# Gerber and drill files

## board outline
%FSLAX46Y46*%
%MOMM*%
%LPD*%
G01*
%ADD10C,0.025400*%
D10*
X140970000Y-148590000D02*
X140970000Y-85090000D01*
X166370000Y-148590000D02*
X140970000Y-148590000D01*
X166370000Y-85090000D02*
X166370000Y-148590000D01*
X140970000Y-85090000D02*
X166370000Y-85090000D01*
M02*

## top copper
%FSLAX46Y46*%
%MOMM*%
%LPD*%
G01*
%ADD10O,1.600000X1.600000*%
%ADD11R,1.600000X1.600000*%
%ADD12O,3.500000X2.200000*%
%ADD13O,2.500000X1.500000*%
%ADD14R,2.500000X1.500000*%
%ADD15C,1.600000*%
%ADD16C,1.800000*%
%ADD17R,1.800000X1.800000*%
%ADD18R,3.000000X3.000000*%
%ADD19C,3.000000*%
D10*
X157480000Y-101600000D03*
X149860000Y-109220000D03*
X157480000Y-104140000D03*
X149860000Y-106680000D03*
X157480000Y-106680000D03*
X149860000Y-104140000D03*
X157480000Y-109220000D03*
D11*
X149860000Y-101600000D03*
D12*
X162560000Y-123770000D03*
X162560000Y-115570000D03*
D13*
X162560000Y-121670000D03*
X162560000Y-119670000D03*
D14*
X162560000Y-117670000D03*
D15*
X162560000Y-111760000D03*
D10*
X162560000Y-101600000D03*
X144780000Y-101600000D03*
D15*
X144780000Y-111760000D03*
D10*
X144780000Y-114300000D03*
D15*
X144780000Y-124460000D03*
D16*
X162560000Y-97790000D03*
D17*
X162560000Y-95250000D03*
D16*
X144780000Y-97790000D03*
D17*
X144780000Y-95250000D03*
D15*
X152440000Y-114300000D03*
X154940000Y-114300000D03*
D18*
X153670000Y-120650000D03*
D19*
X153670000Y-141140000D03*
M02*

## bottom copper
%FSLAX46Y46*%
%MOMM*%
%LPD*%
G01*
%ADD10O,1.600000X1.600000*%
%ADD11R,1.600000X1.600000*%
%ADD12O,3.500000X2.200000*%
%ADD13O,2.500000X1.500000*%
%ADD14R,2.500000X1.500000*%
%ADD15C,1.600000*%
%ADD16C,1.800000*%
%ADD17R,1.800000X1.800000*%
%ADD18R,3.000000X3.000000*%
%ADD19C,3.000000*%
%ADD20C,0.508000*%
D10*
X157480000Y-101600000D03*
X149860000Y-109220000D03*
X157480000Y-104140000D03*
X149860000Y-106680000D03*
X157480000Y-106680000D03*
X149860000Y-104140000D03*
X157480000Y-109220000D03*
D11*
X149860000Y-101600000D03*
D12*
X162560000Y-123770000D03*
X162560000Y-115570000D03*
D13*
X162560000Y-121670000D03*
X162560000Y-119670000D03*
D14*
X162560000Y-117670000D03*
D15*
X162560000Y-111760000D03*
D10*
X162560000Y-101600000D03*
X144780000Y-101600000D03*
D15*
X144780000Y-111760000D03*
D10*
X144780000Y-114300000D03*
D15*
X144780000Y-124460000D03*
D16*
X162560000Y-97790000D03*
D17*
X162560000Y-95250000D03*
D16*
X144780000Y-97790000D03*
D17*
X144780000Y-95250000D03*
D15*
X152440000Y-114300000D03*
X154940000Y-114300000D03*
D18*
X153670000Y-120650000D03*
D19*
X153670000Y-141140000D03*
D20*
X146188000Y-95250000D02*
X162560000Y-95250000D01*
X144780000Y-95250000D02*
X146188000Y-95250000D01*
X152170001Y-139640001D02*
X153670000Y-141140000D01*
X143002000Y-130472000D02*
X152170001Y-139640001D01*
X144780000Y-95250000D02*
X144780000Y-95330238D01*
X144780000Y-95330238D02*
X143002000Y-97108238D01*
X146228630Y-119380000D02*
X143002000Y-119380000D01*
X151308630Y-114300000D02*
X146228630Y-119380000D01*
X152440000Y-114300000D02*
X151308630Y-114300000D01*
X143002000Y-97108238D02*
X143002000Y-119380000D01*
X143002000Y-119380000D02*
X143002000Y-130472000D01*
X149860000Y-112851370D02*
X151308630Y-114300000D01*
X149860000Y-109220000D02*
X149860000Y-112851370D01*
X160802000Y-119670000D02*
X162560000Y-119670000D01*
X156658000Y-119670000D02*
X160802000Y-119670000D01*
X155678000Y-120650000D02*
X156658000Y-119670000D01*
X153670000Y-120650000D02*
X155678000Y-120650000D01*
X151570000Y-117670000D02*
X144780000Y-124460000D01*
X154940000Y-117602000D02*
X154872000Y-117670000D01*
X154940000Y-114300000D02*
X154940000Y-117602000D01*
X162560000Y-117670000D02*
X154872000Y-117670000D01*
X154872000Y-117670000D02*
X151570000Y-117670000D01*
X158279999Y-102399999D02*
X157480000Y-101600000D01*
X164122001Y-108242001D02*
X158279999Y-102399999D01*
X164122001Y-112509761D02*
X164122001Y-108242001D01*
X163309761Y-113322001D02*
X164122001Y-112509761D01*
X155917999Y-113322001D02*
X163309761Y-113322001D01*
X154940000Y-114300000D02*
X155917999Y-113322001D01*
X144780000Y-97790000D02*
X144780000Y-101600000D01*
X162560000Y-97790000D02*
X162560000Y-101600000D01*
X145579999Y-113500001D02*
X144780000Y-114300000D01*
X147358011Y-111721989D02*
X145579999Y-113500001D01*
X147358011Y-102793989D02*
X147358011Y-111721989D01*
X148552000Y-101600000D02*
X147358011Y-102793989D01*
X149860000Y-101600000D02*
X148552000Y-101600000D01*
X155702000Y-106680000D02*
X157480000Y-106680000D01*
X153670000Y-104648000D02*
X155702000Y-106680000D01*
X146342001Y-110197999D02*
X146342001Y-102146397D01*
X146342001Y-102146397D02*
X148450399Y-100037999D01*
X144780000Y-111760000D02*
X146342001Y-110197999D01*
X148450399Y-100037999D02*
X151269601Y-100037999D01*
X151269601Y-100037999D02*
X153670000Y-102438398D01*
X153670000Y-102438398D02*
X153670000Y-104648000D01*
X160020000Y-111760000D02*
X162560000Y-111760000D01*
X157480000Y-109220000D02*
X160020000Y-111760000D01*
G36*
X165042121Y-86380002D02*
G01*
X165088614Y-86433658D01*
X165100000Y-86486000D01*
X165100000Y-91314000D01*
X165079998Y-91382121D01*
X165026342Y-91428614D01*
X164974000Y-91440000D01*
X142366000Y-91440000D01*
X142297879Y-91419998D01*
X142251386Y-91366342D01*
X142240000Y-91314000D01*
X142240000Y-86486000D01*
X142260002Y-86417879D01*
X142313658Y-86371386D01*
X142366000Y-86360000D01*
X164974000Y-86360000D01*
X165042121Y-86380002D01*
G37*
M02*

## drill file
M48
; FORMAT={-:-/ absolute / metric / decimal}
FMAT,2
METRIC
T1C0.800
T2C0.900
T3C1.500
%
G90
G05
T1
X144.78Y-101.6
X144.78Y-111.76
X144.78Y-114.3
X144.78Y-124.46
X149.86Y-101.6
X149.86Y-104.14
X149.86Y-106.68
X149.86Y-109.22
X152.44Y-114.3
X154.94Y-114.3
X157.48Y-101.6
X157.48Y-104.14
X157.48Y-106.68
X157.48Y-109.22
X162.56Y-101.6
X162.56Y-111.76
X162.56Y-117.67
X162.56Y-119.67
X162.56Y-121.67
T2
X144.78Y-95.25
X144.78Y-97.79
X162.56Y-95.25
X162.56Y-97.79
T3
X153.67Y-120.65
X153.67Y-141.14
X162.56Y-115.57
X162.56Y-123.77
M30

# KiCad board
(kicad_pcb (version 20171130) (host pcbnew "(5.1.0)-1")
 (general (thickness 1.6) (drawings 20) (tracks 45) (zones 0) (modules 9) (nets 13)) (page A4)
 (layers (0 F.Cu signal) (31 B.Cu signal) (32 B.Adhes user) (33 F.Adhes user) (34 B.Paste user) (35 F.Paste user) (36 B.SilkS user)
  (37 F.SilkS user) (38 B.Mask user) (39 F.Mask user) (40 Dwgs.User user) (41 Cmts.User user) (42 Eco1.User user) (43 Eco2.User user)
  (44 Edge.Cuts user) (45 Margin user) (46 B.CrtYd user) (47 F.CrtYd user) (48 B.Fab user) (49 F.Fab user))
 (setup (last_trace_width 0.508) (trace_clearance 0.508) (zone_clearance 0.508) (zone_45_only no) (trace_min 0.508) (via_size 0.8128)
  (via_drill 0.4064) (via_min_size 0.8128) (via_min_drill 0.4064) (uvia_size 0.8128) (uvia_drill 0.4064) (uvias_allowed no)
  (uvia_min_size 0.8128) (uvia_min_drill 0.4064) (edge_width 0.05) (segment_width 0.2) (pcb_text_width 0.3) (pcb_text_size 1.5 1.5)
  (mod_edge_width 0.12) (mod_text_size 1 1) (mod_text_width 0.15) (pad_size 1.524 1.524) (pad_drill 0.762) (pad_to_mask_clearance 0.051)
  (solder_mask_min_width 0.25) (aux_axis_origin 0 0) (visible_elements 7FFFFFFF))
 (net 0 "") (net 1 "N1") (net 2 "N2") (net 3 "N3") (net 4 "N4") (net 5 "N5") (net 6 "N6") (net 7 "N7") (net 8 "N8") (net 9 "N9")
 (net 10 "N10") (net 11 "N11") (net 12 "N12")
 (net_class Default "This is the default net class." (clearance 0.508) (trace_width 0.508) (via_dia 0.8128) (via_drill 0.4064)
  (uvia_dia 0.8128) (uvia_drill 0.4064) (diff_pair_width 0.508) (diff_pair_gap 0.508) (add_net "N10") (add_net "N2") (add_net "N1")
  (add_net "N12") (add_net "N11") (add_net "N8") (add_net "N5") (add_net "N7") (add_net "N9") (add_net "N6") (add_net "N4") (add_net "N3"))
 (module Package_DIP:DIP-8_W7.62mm (layer F.Cu) (at 149.86 101.6)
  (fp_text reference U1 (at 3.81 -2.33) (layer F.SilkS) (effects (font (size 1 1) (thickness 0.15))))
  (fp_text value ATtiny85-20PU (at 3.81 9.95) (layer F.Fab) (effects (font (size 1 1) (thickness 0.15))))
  (pad 8 thru_hole oval (at 7.62 0) (size 1.6 1.6) (drill 0.8) (layers *.Cu *.Mask) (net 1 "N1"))
  (pad 4 thru_hole oval (at 0 7.62) (size 1.6 1.6) (drill 0.8) (layers *.Cu *.Mask) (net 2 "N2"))
  (pad 7 thru_hole oval (at 7.62 2.54) (size 1.6 1.6) (drill 0.8) (layers *.Cu *.Mask) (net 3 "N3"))
  (pad 3 thru_hole oval (at 0 5.08) (size 1.6 1.6) (drill 0.8) (layers *.Cu *.Mask) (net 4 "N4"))
  (pad 6 thru_hole oval (at 7.62 5.08) (size 1.6 1.6) (drill 0.8) (layers *.Cu *.Mask) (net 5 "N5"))
  (pad 2 thru_hole oval (at 0 2.54) (size 1.6 1.6) (drill 0.8) (layers *.Cu *.Mask) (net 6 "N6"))
  (pad 5 thru_hole oval (at 7.62 7.62) (size 1.6 1.6) (drill 0.8) (layers *.Cu *.Mask) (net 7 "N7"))
  (pad 1 thru_hole rect (at 0 0) (size 1.6 1.6) (drill 0.8) (layers *.Cu *.Mask) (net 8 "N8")))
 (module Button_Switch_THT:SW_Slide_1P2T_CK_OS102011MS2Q (layer F.Cu) (at 162.56 117.67 270)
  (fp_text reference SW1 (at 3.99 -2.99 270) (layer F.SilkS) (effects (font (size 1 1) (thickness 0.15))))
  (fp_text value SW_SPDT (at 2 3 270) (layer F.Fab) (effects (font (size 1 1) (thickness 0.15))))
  (pad "" thru_hole oval (at 6.1 0 270) (size 2.2 3.5) (drill 1.5) (layers *.Cu *.Mask))
  (pad "" thru_hole oval (at -2.1 0 270) (size 2.2 3.5) (drill 1.5) (layers *.Cu *.Mask))
  (pad 3 thru_hole oval (at 4 0 270) (size 1.5 2.5) (drill 0.8) (layers *.Cu *.Mask) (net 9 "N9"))
  (pad 2 thru_hole oval (at 2 0 270) (size 1.5 2.5) (drill 0.8) (layers *.Cu *.Mask) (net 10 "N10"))
  (pad 1 thru_hole rect (at 0 0 270) (size 1.5 2.5) (drill 0.8) (layers *.Cu *.Mask) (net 1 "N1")))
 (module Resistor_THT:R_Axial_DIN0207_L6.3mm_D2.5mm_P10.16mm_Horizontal (layer F.Cu) (at 162.56 111.76 90)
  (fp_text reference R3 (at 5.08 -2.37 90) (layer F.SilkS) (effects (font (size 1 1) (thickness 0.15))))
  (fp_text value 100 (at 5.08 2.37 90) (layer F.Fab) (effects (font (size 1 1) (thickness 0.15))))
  (pad 1 thru_hole circle (at 0 0 90) (size 1.6 1.6) (drill 0.8) (layers *.Cu *.Mask) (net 7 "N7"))
  (pad 2 thru_hole oval (at 10.16 0 90) (size 1.6 1.6) (drill 0.8) (layers *.Cu *.Mask) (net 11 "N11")))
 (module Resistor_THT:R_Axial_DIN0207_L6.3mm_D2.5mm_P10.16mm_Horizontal (layer F.Cu) (at 144.78 111.76 90)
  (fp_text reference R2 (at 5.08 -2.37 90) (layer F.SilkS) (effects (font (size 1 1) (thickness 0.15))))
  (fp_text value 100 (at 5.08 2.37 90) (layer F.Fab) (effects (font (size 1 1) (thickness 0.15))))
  (pad 2 thru_hole oval (at 10.16 0 90) (size 1.6 1.6) (drill 0.8) (layers *.Cu *.Mask) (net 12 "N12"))
  (pad 1 thru_hole circle (at 0 0 90) (size 1.6 1.6) (drill 0.8) (layers *.Cu *.Mask) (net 5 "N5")))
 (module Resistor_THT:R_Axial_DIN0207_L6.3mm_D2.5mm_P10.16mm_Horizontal (layer F.Cu) (at 144.78 124.46 90)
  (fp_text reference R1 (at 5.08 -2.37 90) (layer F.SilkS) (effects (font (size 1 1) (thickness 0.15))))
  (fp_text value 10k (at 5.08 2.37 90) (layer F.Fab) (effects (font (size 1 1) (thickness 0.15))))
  (pad 2 thru_hole oval (at 10.16 0 90) (size 1.6 1.6) (drill 0.8) (layers *.Cu *.Mask) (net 8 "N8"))
  (pad 1 thru_hole circle (at 0 0 90) (size 1.6 1.6) (drill 0.8) (layers *.Cu *.Mask) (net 1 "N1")))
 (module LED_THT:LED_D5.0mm (layer F.Cu) (at 162.56 95.25 270)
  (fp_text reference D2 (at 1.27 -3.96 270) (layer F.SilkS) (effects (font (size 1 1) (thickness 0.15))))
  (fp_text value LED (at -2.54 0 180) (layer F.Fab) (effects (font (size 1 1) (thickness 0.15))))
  (pad 2 thru_hole circle (at 2.54 0 270) (size 1.8 1.8) (drill 0.9) (layers *.Cu *.Mask) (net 11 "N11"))
  (pad 1 thru_hole rect (at 0 0 270) (size 1.8 1.8) (drill 0.9) (layers *.Cu *.Mask) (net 2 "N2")))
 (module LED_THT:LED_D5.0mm (layer F.Cu) (at 144.78 95.25 270)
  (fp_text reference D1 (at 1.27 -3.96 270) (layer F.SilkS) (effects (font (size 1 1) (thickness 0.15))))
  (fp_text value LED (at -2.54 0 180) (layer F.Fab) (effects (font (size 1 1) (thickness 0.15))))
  (pad 2 thru_hole circle (at 2.54 0 270) (size 1.8 1.8) (drill 0.9) (layers *.Cu *.Mask) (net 12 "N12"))
  (pad 1 thru_hole rect (at 0 0 270) (size 1.8 1.8) (drill 0.9) (layers *.Cu *.Mask) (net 2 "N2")))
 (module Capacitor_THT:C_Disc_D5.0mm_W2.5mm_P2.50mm (layer F.Cu) (at 154.94 114.3 180)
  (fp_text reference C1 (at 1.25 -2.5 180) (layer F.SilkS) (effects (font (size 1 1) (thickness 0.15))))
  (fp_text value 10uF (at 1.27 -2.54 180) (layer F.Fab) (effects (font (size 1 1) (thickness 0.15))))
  (pad 2 thru_hole circle (at 2.5 0 180) (size 1.6 1.6) (drill 0.8) (layers *.Cu *.Mask) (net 2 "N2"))
  (pad 1 thru_hole circle (at 0 0 180) (size 1.6 1.6) (drill 0.8) (layers *.Cu *.Mask) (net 1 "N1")))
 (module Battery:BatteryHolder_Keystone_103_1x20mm (layer F.Cu) (at 153.67 120.65 270)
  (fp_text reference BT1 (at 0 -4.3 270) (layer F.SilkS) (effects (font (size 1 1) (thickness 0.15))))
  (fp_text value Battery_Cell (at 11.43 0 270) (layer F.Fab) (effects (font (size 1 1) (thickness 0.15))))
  (pad 1 thru_hole rect (at 0 0 270) (size 3 3) (drill 1.5) (layers *.Cu *.Mask) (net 10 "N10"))
  (pad 2 thru_hole circle (at 20.49 0 270) (size 3 3) (drill 1.5) (layers *.Cu *.Mask) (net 2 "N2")))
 (gr_line (start 140.97 148.59) (end 140.97 85.09) (layer Edge.Cuts) (width 0.0254))
 (gr_line (start 166.37 148.59) (end 140.97 148.59) (layer Edge.Cuts) (width 0.0254))
 (gr_line (start 166.37 85.09) (end 166.37 148.59) (layer Edge.Cuts) (width 0.0254))
 (gr_line (start 140.97 85.09) (end 166.37 85.09) (layer Edge.Cuts) (width 0.0254))
 (segment (start 146.188 95.25) (end 162.56 95.25) (width 0.508) (layer B.Cu) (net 2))
 (segment (start 144.78 95.25) (end 146.188 95.25) (width 0.508) (layer B.Cu) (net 2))
 (segment (start 152.170001 139.640001) (end 153.67 141.14) (width 0.508) (layer B.Cu) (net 2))
 (segment (start 143.002 130.472) (end 152.170001 139.640001) (width 0.508) (layer B.Cu) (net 2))
 (segment (start 144.78 95.25) (end 144.78 95.330238) (width 0.508) (layer B.Cu) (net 2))
 (segment (start 144.78 95.330238) (end 143.002 97.108238) (width 0.508) (layer B.Cu) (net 2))
 (segment (start 146.22863 119.38) (end 143.002 119.38) (width 0.508) (layer B.Cu) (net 2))
 (segment (start 151.30863 114.3) (end 146.22863 119.38) (width 0.508) (layer B.Cu) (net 2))
 (segment (start 152.44 114.3) (end 151.30863 114.3) (width 0.508) (layer B.Cu) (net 2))
 (segment (start 143.002 97.108238) (end 143.002 119.38) (width 0.508) (layer B.Cu) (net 2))
 (segment (start 143.002 119.38) (end 143.002 130.472) (width 0.508) (layer B.Cu) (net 2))
 (segment (start 149.86 112.85137) (end 151.30863 114.3) (width 0.508) (layer B.Cu) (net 2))
 (segment (start 149.86 109.22) (end 149.86 112.85137) (width 0.508) (layer B.Cu) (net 2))
 (segment (start 160.802 119.67) (end 162.56 119.67) (width 0.508) (layer B.Cu) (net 10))
 (segment (start 156.658 119.67) (end 160.802 119.67) (width 0.508) (layer B.Cu) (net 10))
 (segment (start 155.678 120.65) (end 156.658 119.67) (width 0.508) (layer B.Cu) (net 10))
 (segment (start 153.67 120.65) (end 155.678 120.65) (width 0.508) (layer B.Cu) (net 10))
 (segment (start 151.57 117.67) (end 144.78 124.46) (width 0.508) (layer B.Cu) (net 1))
 (segment (start 154.94 117.602) (end 154.872 117.67) (width 0.508) (layer B.Cu) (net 1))
 (segment (start 154.94 114.3) (end 154.94 117.602) (width 0.508) (layer B.Cu) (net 1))
 (segment (start 162.56 117.67) (end 154.872 117.67) (width 0.508) (layer B.Cu) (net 1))
 (segment (start 154.872 117.67) (end 151.57 117.67) (width 0.508) (layer B.Cu) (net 1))
 (segment (start 158.279999 102.399999) (end 157.48 101.6) (width 0.508) (layer B.Cu) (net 1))
 (segment (start 164.122001 108.242001) (end 158.279999 102.399999) (width 0.508) (layer B.Cu) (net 1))
 (segment (start 164.122001 112.509761) (end 164.122001 108.242001) (width 0.508) (layer B.Cu) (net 1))
 (segment (start 163.309761 113.322001) (end 164.122001 112.509761) (width 0.508) (layer B.Cu) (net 1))
 (segment (start 155.917999 113.322001) (end 163.309761 113.322001) (width 0.508) (layer B.Cu) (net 1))
 (segment (start 154.94 114.3) (end 155.917999 113.322001) (width 0.508) (layer B.Cu) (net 1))
 (segment (start 144.78 97.79) (end 144.78 101.6) (width 0.508) (layer B.Cu) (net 12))
 (segment (start 162.56 97.79) (end 162.56 101.6) (width 0.508) (layer B.Cu) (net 11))
 (segment (start 145.579999 113.500001) (end 144.78 114.3) (width 0.508) (layer B.Cu) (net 8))
 (segment (start 147.358011 111.721989) (end 145.579999 113.500001) (width 0.508) (layer B.Cu) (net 8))
 (segment (start 147.358011 102.793989) (end 147.358011 111.721989) (width 0.508) (layer B.Cu) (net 8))
 (segment (start 148.552 101.6) (end 147.358011 102.793989) (width 0.508) (layer B.Cu) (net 8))
 (segment (start 149.86 101.6) (end 148.552 101.6) (width 0.508) (layer B.Cu) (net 8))
 (segment (start 155.702 106.68) (end 157.48 106.68) (width 0.508) (layer B.Cu) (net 5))
 (segment (start 153.67 104.648) (end 155.702 106.68) (width 0.508) (layer B.Cu) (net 5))
 (segment (start 146.342001 110.197999) (end 146.342001 102.146397) (width 0.508) (layer B.Cu) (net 5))
 (segment (start 146.342001 102.146397) (end 148.450399 100.037999) (width 0.508) (layer B.Cu) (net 5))
 (segment (start 144.78 111.76) (end 146.342001 110.197999) (width 0.508) (layer B.Cu) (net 5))
 (segment (start 148.450399 100.037999) (end 151.269601 100.037999) (width 0.508) (layer B.Cu) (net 5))
 (segment (start 151.269601 100.037999) (end 153.67 102.438398) (width 0.508) (layer B.Cu) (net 5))
 (segment (start 153.67 102.438398) (end 153.67 104.648) (width 0.508) (layer B.Cu) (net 5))
 (segment (start 160.02 111.76) (end 162.56 111.76) (width 0.508) (layer B.Cu) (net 7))
 (segment (start 157.48 109.22) (end 160.02 111.76) (width 0.508) (layer B.Cu) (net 7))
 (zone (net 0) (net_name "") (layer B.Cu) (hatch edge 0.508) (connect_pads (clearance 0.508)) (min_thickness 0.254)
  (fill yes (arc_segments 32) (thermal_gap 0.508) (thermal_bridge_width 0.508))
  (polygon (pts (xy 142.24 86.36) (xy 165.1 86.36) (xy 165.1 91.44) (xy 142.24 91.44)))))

